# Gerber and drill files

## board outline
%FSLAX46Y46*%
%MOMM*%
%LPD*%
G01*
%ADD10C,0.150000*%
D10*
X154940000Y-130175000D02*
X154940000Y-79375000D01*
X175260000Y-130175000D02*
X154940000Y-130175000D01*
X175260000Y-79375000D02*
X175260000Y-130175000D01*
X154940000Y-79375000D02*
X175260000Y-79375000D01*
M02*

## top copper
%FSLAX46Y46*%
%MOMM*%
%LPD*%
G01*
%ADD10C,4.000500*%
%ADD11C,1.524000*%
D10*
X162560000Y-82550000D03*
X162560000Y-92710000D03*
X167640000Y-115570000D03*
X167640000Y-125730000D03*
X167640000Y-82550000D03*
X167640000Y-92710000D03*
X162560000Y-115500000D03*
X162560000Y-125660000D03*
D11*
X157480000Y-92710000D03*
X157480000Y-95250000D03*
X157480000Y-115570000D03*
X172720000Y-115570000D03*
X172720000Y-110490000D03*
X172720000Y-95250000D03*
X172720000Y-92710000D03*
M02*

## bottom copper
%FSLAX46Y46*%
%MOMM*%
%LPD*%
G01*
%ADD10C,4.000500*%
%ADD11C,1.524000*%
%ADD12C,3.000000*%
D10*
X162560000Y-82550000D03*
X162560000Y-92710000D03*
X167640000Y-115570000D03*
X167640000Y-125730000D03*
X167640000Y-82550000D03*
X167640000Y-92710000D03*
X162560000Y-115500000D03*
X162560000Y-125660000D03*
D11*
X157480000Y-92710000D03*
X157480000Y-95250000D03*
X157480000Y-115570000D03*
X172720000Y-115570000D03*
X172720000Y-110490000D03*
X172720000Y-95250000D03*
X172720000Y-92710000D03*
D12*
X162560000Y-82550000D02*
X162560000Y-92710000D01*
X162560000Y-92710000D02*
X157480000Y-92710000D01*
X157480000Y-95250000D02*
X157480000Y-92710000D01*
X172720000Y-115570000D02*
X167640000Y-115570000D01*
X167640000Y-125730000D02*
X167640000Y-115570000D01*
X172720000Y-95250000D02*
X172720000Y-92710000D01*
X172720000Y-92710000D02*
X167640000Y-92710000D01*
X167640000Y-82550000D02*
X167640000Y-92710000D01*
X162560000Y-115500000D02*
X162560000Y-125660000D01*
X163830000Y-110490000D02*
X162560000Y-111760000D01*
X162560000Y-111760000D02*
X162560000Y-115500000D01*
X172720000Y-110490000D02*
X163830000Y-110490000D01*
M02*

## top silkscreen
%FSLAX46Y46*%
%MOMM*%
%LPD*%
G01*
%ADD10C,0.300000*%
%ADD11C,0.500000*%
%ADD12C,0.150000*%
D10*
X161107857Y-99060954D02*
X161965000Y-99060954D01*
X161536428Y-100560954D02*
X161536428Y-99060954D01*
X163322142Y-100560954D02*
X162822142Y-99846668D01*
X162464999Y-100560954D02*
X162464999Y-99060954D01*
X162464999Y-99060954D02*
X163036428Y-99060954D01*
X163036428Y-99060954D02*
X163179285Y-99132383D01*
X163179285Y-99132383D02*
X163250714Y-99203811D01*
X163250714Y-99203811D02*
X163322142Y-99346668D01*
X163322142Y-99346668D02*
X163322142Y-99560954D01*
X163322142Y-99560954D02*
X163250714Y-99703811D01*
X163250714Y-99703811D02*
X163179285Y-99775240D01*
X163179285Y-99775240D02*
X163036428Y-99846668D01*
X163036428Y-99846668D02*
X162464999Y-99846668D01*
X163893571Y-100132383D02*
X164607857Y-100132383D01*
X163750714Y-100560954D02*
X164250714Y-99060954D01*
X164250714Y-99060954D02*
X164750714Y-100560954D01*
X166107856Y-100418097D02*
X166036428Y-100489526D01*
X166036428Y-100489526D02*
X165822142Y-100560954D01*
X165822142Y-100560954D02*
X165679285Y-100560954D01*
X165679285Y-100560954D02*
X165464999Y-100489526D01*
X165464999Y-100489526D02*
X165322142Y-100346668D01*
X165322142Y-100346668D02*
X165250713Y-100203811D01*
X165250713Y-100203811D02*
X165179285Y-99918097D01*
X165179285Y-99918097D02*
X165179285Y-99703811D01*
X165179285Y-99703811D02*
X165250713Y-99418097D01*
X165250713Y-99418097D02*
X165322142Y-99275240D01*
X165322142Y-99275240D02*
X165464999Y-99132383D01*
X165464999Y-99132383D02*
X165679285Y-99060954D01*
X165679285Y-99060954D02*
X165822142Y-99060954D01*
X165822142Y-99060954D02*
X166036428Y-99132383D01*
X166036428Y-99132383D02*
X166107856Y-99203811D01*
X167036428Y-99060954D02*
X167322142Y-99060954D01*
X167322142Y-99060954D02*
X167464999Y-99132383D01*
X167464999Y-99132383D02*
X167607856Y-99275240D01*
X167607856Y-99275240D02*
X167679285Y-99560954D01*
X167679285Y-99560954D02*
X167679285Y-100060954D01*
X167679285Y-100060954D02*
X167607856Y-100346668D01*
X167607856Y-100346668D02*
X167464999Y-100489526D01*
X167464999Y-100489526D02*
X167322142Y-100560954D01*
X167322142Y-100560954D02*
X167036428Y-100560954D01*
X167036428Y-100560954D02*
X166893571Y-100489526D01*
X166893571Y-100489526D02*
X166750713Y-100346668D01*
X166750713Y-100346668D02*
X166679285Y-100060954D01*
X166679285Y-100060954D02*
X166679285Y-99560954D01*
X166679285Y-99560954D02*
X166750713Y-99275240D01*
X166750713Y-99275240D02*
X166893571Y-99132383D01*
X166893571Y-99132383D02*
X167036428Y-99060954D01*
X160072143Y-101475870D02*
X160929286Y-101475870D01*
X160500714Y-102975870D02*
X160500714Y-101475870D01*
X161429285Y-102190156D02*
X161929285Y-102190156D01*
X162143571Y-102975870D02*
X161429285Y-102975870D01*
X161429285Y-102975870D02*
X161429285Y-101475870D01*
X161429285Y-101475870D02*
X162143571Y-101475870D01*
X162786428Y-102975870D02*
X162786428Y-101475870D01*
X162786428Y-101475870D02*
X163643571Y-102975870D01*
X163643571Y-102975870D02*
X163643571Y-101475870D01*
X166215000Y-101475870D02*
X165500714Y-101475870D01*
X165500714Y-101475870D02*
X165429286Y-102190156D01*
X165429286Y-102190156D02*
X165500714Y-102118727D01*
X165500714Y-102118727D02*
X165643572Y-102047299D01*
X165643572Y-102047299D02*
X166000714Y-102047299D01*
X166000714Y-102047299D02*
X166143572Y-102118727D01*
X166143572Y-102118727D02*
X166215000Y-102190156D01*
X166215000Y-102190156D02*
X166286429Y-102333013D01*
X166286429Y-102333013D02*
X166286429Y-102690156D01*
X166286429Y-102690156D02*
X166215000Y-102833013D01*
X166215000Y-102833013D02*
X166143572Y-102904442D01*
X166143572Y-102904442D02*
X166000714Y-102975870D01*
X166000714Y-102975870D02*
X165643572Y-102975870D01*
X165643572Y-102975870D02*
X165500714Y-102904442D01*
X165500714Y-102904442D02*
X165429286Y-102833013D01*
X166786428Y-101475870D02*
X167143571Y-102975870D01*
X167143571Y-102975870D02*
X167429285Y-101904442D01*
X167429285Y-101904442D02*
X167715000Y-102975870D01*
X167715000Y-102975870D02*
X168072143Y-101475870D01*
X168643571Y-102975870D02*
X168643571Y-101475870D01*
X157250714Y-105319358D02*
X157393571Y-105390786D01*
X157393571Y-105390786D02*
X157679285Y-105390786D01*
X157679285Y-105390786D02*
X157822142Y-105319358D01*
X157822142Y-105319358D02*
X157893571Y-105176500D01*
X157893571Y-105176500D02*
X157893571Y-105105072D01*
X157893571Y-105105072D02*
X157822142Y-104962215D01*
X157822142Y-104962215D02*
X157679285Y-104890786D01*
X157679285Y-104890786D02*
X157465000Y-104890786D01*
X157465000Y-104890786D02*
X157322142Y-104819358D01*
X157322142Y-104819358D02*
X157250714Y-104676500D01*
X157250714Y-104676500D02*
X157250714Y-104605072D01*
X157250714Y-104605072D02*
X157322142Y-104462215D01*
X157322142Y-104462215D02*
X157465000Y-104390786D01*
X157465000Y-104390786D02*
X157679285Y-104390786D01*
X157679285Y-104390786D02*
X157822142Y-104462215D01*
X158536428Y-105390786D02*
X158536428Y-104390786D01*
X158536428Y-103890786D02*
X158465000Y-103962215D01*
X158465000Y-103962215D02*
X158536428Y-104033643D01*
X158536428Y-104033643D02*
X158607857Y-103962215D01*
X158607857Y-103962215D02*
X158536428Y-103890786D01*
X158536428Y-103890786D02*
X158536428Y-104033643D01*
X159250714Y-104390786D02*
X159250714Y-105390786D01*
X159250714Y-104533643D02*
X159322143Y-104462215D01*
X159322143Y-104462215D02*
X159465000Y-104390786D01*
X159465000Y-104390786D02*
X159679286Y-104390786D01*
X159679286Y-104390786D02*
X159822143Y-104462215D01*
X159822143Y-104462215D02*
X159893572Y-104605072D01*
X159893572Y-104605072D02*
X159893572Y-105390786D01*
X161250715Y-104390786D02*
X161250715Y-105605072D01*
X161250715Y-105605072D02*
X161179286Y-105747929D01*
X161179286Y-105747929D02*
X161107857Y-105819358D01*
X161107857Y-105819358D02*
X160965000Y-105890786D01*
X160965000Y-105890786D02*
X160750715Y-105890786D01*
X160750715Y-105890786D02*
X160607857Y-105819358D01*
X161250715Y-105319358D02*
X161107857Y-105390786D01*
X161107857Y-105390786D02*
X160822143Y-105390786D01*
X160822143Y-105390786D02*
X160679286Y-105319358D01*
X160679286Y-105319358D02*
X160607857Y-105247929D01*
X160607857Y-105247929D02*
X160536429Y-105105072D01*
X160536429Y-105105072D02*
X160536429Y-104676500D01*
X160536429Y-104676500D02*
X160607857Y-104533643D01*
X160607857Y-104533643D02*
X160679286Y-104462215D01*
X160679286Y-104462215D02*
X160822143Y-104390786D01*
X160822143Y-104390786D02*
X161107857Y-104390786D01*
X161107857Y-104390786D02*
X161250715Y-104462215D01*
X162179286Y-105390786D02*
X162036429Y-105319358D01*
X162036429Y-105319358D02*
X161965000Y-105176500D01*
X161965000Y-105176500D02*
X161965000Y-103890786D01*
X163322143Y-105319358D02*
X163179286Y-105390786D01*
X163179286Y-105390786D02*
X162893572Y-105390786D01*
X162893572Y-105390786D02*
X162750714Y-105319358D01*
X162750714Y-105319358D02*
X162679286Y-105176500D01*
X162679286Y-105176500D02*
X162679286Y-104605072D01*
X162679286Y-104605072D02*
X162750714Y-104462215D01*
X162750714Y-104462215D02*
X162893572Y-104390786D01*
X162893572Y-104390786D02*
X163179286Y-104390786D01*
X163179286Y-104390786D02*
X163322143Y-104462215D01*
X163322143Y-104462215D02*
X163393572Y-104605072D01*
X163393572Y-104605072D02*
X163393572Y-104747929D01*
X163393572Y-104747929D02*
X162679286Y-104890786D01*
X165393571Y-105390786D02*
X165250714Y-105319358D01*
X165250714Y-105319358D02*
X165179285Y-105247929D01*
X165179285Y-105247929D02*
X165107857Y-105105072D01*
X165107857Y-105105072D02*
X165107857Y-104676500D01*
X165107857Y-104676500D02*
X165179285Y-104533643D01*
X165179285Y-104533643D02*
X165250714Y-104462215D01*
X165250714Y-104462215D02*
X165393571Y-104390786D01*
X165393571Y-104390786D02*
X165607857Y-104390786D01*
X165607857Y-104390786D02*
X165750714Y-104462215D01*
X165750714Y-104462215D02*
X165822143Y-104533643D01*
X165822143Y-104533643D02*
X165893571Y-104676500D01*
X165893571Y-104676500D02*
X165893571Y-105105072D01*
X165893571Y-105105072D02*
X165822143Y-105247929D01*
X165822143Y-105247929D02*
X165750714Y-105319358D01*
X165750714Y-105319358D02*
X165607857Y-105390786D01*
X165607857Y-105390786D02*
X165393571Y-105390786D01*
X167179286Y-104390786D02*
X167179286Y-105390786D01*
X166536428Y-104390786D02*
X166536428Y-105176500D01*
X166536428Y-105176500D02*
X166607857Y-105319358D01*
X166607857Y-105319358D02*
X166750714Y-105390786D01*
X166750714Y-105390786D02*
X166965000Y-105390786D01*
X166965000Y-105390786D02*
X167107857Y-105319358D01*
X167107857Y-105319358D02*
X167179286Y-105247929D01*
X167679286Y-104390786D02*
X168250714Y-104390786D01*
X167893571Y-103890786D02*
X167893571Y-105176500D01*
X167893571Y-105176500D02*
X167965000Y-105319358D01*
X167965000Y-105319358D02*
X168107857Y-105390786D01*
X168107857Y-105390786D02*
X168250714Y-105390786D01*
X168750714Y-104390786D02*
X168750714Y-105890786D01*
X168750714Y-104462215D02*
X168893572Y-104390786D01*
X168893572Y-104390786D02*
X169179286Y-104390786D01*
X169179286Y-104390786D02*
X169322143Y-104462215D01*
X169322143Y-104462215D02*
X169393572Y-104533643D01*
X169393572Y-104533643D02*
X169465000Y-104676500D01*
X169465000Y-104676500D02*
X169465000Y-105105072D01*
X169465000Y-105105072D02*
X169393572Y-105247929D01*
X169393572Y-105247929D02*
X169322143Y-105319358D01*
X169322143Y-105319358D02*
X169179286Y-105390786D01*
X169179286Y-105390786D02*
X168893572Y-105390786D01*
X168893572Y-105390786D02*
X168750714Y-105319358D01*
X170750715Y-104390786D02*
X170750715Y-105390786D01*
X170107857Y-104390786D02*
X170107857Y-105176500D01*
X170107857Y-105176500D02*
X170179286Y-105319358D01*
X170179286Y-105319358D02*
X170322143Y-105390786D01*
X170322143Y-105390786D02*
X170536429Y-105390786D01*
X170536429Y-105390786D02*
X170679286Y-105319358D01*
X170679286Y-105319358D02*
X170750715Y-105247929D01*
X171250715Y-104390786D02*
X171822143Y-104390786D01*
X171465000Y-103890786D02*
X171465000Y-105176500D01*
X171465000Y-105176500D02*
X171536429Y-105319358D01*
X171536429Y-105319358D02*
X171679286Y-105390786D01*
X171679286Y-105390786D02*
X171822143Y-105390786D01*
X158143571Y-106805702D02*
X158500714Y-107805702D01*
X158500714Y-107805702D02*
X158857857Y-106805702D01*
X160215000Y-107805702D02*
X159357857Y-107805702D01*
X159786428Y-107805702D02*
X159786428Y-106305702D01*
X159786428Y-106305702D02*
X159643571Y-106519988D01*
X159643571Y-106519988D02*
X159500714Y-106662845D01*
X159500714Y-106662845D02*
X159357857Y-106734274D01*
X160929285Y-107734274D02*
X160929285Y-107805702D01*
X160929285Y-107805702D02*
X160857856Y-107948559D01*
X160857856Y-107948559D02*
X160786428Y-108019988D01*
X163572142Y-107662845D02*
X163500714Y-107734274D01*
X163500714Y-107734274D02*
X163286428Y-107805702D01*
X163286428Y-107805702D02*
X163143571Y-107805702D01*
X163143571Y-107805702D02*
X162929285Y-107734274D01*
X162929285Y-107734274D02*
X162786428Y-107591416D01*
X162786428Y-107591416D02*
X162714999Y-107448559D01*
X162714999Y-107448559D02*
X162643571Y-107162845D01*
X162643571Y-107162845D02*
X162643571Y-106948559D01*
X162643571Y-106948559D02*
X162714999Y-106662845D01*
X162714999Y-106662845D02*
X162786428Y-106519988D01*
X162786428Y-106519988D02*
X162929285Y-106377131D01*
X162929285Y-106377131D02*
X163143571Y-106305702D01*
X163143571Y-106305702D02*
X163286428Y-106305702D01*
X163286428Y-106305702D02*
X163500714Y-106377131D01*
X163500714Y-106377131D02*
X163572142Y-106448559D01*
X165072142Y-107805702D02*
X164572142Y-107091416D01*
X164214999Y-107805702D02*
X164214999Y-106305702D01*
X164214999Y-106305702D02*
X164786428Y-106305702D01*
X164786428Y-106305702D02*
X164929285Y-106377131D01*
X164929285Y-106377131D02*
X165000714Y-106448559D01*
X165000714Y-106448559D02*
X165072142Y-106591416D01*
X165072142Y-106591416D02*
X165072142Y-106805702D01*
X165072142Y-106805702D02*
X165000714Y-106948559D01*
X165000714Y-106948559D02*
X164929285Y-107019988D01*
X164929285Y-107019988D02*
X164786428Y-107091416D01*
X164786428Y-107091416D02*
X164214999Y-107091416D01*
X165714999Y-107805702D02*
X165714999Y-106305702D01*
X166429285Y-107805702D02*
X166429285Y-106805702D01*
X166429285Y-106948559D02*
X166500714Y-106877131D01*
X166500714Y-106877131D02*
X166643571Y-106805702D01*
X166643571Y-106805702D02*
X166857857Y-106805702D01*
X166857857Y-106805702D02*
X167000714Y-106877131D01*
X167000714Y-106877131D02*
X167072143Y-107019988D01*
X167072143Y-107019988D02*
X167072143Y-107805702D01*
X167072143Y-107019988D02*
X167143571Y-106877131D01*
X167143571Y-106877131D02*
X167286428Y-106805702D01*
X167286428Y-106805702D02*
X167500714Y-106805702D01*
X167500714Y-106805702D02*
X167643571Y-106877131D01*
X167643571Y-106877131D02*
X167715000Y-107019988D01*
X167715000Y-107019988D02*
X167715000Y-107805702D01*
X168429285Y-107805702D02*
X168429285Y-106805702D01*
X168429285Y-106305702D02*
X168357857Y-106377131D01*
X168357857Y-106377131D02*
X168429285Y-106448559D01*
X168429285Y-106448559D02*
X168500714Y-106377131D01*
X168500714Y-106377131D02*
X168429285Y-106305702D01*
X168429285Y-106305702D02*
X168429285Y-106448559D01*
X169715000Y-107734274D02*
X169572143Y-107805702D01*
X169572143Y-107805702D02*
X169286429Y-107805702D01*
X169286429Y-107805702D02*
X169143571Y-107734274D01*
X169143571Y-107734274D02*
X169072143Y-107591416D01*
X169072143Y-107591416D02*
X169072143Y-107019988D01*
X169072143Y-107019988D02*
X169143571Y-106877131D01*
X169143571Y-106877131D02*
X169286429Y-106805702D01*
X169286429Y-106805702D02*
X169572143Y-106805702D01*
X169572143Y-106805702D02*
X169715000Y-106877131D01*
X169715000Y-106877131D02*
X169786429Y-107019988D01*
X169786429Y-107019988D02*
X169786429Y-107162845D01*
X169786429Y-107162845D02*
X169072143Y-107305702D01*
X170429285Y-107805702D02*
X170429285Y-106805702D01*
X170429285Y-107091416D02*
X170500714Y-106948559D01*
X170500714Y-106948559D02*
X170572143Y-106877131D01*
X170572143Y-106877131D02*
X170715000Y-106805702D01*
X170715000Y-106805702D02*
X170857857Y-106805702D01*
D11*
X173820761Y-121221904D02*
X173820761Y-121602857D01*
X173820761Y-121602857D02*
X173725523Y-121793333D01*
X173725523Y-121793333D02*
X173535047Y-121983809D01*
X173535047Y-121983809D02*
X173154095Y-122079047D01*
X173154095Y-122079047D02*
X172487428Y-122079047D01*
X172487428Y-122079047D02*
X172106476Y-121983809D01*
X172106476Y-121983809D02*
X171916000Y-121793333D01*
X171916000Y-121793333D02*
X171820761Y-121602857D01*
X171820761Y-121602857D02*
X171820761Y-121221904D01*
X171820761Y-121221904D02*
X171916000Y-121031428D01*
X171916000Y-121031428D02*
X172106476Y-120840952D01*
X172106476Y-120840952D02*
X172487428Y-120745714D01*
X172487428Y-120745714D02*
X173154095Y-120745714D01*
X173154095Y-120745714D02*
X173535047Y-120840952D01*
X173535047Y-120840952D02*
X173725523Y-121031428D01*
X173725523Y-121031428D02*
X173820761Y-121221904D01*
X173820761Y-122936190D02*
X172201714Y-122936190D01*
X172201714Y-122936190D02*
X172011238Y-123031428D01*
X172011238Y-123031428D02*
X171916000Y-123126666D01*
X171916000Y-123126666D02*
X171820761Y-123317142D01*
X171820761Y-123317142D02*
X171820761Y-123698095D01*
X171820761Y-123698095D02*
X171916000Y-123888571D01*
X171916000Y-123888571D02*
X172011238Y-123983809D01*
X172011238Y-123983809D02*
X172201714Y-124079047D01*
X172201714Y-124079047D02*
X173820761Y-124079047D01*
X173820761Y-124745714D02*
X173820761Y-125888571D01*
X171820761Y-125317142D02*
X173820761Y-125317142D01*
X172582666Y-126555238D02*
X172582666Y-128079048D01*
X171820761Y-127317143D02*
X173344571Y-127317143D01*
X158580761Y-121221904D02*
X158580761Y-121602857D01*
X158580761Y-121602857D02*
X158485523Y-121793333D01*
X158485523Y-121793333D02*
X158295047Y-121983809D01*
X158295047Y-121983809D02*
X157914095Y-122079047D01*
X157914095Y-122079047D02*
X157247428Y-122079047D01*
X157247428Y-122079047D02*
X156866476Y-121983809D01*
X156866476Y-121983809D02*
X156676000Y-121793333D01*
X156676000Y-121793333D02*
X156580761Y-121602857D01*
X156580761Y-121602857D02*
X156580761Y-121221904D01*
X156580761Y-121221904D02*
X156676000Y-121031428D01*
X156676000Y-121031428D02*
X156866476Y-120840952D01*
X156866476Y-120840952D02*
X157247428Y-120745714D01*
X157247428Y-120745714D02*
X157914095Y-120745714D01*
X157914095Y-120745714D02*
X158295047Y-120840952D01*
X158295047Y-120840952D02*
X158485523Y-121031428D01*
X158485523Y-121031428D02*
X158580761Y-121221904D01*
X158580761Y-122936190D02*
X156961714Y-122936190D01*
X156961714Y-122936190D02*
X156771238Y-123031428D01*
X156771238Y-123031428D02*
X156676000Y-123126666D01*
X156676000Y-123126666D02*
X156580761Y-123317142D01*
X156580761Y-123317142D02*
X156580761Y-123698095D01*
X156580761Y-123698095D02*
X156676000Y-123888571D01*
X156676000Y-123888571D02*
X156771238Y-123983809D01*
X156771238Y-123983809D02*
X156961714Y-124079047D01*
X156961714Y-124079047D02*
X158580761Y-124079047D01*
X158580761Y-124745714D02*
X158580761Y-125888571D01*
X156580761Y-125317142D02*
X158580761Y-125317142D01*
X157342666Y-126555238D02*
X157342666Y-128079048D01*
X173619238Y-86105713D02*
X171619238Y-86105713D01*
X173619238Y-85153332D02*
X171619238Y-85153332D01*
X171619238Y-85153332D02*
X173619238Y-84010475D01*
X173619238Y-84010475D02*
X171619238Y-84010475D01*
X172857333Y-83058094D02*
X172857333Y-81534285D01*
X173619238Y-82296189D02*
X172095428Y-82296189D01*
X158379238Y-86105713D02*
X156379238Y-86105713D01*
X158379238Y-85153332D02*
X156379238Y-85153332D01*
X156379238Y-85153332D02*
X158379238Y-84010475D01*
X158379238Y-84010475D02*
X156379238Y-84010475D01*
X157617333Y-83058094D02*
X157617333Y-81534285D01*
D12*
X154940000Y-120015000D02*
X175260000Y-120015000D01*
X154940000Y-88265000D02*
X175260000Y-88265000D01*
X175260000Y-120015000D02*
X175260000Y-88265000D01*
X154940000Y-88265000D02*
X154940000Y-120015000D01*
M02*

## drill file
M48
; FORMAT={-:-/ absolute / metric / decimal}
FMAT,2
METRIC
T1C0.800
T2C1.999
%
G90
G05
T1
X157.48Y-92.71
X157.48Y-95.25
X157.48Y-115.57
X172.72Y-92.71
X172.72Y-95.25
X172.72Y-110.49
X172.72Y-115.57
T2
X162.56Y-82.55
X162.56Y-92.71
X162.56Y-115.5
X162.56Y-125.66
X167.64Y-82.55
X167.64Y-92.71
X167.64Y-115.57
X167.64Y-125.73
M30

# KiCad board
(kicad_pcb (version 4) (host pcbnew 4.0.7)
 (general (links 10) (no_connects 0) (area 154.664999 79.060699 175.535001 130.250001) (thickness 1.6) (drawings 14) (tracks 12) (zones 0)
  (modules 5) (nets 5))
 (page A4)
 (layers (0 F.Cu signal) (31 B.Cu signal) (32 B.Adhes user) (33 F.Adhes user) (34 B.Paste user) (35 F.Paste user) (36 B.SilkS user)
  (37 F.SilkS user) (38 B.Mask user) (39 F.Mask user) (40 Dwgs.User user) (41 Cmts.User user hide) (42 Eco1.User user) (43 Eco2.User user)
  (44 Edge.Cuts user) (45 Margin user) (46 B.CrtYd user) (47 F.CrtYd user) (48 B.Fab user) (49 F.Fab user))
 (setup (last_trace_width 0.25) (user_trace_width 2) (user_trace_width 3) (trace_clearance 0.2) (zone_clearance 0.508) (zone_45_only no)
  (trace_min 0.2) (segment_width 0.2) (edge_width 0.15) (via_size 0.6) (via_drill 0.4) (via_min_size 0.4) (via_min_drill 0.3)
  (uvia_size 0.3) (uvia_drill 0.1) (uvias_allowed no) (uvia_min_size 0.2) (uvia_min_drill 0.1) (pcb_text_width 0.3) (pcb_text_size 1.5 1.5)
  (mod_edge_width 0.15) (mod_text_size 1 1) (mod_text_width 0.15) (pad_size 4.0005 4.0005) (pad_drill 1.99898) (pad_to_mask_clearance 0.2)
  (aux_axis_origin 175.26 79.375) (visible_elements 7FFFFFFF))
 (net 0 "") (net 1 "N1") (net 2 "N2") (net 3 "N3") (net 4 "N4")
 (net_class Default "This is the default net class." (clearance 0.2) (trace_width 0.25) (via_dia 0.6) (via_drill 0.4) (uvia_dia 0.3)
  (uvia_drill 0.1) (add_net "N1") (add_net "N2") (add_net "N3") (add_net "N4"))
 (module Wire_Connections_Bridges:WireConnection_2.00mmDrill (layer F.Cu) (at 162.56 82.55 270)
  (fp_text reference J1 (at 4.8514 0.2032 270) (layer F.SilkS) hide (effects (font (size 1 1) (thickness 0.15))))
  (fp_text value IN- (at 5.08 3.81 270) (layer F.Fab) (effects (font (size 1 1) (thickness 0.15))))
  (pad 1 thru_hole circle (at 0 0 270) (size 4.0005 4.0005) (drill 1.99898) (layers *.Cu *.Mask) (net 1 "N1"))
  (pad 2 thru_hole circle (at 10.16 0 270) (size 4.0005 4.0005) (drill 1.99898) (layers *.Cu B.Mask) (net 1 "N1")))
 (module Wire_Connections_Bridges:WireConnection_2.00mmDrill (layer F.Cu) (at 167.64 115.57 270)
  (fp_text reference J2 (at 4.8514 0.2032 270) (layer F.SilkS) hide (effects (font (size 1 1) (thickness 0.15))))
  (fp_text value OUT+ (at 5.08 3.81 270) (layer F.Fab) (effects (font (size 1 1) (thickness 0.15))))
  (pad 1 thru_hole circle (at 0 0 270) (size 4.0005 4.0005) (drill 1.99898) (layers *.Cu B.Mask) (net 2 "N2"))
  (pad 2 thru_hole circle (at 10.16 0 270) (size 4.0005 4.0005) (drill 1.99898) (layers *.Cu *.Mask) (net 2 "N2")))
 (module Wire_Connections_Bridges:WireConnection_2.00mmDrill (layer F.Cu) (at 167.64 82.55 270)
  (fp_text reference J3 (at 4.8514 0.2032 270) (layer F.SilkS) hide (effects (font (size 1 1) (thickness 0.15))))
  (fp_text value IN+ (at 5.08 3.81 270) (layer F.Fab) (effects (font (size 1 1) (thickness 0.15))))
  (pad 1 thru_hole circle (at 0 0 270) (size 4.0005 4.0005) (drill 1.99898) (layers *.Cu *.Mask) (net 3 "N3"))
  (pad 2 thru_hole circle (at 10.16 0 270) (size 4.0005 4.0005) (drill 1.99898) (layers *.Cu B.Mask) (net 3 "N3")))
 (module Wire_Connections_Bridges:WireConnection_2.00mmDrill (layer F.Cu) (at 162.56 115.5 270)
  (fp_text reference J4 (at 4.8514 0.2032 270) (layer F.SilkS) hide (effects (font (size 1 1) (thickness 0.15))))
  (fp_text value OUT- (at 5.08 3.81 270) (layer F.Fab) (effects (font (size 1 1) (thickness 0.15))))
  (pad 1 thru_hole circle (at 0 0 270) (size 4.0005 4.0005) (drill 1.99898) (layers *.Cu B.Mask) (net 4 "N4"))
  (pad 2 thru_hole circle (at 10.16 0 270) (size 4.0005 4.0005) (drill 1.99898) (layers *.Cu *.Mask) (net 4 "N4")))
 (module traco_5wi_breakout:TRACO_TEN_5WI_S (layer F.Cu) (at 165.1 104.14)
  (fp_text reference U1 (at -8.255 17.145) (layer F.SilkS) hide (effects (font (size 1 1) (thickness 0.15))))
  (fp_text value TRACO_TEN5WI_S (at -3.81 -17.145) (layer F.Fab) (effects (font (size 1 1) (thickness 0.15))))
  (fp_line (start -10.16 15.875) (end 10.16 15.875) (layer F.SilkS) (width 0.15))
  (fp_line (start -10.16 -15.875) (end 10.16 -15.875) (layer F.SilkS) (width 0.15))
  (fp_line (start 10.16 15.875) (end 10.16 -15.875) (layer F.SilkS) (width 0.15))
  (fp_line (start -10.16 -15.875) (end -10.16 15.875) (layer F.SilkS) (width 0.15))
  (pad 2 thru_hole circle (at -7.62 -11.43) (size 1.524 1.524) (drill 0.8) (layers *.Cu *.Mask) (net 1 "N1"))
  (pad 3 thru_hole circle (at -7.62 -8.89) (size 1.524 1.524) (drill 0.8) (layers *.Cu *.Mask) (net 1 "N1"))
  (pad 11 thru_hole circle (at -7.62 11.43) (size 1.524 1.524) (drill 0.8) (layers *.Cu *.Mask))
  (pad 14 thru_hole circle (at 7.62 11.43) (size 1.524 1.524) (drill 0.8) (layers *.Cu *.Mask) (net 2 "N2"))
  (pad 16 thru_hole circle (at 7.62 6.35) (size 1.524 1.524) (drill 0.8) (layers *.Cu *.Mask) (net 4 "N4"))
  (pad 22 thru_hole circle (at 7.62 -8.89) (size 1.524 1.524) (drill 0.8) (layers *.Cu *.Mask) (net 3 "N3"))
  (pad 23 thru_hole circle (at 7.62 -11.43) (size 1.524 1.524) (drill 0.8) (layers *.Cu *.Mask) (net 3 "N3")))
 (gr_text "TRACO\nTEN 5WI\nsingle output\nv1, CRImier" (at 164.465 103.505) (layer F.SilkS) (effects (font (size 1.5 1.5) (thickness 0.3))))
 (gr_line (start 154.94 130.175) (end 154.94 79.375) (layer Edge.Cuts) (width 0.15))
 (gr_line (start 175.26 130.175) (end 154.94 130.175) (layer Edge.Cuts) (width 0.15))
 (gr_line (start 175.26 79.375) (end 175.26 130.175) (layer Edge.Cuts) (width 0.15))
 (gr_line (start 154.94 79.375) (end 175.26 79.375) (layer Edge.Cuts) (width 0.15))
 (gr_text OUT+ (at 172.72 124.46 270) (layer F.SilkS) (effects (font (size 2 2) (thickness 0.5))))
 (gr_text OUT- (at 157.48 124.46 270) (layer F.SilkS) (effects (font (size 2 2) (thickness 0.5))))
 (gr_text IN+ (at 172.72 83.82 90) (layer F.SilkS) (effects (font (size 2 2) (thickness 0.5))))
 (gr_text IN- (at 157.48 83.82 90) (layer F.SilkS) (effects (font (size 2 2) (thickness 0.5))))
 (segment (start 162.56 82.55) (end 162.56 92.71) (width 3) (layer B.Cu) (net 1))
 (segment (start 162.56 92.71) (end 157.48 92.71) (width 3) (layer B.Cu) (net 1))
 (segment (start 157.48 95.25) (end 157.48 92.71) (width 3) (layer B.Cu) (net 1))
 (segment (start 172.72 115.57) (end 167.64 115.57) (width 3) (layer B.Cu) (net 2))
 (segment (start 167.64 125.73) (end 167.64 115.57) (width 3) (layer B.Cu) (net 2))
 (segment (start 172.72 95.25) (end 172.72 92.71) (width 3) (layer B.Cu) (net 3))
 (segment (start 172.72 92.71) (end 167.64 92.71) (width 3) (layer B.Cu) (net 3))
 (segment (start 167.64 82.55) (end 167.64 92.71) (width 3) (layer B.Cu) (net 3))
 (segment (start 162.56 115.5) (end 162.56 125.66) (width 3) (layer B.Cu) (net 4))
 (segment (start 163.83 110.49) (end 162.56 111.76) (width 3) (layer B.Cu) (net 4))
 (segment (start 162.56 111.76) (end 162.56 115.5) (width 3) (layer B.Cu) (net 4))
 (segment (start 172.72 110.49) (end 163.83 110.49) (width 3) (layer B.Cu) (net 4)))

